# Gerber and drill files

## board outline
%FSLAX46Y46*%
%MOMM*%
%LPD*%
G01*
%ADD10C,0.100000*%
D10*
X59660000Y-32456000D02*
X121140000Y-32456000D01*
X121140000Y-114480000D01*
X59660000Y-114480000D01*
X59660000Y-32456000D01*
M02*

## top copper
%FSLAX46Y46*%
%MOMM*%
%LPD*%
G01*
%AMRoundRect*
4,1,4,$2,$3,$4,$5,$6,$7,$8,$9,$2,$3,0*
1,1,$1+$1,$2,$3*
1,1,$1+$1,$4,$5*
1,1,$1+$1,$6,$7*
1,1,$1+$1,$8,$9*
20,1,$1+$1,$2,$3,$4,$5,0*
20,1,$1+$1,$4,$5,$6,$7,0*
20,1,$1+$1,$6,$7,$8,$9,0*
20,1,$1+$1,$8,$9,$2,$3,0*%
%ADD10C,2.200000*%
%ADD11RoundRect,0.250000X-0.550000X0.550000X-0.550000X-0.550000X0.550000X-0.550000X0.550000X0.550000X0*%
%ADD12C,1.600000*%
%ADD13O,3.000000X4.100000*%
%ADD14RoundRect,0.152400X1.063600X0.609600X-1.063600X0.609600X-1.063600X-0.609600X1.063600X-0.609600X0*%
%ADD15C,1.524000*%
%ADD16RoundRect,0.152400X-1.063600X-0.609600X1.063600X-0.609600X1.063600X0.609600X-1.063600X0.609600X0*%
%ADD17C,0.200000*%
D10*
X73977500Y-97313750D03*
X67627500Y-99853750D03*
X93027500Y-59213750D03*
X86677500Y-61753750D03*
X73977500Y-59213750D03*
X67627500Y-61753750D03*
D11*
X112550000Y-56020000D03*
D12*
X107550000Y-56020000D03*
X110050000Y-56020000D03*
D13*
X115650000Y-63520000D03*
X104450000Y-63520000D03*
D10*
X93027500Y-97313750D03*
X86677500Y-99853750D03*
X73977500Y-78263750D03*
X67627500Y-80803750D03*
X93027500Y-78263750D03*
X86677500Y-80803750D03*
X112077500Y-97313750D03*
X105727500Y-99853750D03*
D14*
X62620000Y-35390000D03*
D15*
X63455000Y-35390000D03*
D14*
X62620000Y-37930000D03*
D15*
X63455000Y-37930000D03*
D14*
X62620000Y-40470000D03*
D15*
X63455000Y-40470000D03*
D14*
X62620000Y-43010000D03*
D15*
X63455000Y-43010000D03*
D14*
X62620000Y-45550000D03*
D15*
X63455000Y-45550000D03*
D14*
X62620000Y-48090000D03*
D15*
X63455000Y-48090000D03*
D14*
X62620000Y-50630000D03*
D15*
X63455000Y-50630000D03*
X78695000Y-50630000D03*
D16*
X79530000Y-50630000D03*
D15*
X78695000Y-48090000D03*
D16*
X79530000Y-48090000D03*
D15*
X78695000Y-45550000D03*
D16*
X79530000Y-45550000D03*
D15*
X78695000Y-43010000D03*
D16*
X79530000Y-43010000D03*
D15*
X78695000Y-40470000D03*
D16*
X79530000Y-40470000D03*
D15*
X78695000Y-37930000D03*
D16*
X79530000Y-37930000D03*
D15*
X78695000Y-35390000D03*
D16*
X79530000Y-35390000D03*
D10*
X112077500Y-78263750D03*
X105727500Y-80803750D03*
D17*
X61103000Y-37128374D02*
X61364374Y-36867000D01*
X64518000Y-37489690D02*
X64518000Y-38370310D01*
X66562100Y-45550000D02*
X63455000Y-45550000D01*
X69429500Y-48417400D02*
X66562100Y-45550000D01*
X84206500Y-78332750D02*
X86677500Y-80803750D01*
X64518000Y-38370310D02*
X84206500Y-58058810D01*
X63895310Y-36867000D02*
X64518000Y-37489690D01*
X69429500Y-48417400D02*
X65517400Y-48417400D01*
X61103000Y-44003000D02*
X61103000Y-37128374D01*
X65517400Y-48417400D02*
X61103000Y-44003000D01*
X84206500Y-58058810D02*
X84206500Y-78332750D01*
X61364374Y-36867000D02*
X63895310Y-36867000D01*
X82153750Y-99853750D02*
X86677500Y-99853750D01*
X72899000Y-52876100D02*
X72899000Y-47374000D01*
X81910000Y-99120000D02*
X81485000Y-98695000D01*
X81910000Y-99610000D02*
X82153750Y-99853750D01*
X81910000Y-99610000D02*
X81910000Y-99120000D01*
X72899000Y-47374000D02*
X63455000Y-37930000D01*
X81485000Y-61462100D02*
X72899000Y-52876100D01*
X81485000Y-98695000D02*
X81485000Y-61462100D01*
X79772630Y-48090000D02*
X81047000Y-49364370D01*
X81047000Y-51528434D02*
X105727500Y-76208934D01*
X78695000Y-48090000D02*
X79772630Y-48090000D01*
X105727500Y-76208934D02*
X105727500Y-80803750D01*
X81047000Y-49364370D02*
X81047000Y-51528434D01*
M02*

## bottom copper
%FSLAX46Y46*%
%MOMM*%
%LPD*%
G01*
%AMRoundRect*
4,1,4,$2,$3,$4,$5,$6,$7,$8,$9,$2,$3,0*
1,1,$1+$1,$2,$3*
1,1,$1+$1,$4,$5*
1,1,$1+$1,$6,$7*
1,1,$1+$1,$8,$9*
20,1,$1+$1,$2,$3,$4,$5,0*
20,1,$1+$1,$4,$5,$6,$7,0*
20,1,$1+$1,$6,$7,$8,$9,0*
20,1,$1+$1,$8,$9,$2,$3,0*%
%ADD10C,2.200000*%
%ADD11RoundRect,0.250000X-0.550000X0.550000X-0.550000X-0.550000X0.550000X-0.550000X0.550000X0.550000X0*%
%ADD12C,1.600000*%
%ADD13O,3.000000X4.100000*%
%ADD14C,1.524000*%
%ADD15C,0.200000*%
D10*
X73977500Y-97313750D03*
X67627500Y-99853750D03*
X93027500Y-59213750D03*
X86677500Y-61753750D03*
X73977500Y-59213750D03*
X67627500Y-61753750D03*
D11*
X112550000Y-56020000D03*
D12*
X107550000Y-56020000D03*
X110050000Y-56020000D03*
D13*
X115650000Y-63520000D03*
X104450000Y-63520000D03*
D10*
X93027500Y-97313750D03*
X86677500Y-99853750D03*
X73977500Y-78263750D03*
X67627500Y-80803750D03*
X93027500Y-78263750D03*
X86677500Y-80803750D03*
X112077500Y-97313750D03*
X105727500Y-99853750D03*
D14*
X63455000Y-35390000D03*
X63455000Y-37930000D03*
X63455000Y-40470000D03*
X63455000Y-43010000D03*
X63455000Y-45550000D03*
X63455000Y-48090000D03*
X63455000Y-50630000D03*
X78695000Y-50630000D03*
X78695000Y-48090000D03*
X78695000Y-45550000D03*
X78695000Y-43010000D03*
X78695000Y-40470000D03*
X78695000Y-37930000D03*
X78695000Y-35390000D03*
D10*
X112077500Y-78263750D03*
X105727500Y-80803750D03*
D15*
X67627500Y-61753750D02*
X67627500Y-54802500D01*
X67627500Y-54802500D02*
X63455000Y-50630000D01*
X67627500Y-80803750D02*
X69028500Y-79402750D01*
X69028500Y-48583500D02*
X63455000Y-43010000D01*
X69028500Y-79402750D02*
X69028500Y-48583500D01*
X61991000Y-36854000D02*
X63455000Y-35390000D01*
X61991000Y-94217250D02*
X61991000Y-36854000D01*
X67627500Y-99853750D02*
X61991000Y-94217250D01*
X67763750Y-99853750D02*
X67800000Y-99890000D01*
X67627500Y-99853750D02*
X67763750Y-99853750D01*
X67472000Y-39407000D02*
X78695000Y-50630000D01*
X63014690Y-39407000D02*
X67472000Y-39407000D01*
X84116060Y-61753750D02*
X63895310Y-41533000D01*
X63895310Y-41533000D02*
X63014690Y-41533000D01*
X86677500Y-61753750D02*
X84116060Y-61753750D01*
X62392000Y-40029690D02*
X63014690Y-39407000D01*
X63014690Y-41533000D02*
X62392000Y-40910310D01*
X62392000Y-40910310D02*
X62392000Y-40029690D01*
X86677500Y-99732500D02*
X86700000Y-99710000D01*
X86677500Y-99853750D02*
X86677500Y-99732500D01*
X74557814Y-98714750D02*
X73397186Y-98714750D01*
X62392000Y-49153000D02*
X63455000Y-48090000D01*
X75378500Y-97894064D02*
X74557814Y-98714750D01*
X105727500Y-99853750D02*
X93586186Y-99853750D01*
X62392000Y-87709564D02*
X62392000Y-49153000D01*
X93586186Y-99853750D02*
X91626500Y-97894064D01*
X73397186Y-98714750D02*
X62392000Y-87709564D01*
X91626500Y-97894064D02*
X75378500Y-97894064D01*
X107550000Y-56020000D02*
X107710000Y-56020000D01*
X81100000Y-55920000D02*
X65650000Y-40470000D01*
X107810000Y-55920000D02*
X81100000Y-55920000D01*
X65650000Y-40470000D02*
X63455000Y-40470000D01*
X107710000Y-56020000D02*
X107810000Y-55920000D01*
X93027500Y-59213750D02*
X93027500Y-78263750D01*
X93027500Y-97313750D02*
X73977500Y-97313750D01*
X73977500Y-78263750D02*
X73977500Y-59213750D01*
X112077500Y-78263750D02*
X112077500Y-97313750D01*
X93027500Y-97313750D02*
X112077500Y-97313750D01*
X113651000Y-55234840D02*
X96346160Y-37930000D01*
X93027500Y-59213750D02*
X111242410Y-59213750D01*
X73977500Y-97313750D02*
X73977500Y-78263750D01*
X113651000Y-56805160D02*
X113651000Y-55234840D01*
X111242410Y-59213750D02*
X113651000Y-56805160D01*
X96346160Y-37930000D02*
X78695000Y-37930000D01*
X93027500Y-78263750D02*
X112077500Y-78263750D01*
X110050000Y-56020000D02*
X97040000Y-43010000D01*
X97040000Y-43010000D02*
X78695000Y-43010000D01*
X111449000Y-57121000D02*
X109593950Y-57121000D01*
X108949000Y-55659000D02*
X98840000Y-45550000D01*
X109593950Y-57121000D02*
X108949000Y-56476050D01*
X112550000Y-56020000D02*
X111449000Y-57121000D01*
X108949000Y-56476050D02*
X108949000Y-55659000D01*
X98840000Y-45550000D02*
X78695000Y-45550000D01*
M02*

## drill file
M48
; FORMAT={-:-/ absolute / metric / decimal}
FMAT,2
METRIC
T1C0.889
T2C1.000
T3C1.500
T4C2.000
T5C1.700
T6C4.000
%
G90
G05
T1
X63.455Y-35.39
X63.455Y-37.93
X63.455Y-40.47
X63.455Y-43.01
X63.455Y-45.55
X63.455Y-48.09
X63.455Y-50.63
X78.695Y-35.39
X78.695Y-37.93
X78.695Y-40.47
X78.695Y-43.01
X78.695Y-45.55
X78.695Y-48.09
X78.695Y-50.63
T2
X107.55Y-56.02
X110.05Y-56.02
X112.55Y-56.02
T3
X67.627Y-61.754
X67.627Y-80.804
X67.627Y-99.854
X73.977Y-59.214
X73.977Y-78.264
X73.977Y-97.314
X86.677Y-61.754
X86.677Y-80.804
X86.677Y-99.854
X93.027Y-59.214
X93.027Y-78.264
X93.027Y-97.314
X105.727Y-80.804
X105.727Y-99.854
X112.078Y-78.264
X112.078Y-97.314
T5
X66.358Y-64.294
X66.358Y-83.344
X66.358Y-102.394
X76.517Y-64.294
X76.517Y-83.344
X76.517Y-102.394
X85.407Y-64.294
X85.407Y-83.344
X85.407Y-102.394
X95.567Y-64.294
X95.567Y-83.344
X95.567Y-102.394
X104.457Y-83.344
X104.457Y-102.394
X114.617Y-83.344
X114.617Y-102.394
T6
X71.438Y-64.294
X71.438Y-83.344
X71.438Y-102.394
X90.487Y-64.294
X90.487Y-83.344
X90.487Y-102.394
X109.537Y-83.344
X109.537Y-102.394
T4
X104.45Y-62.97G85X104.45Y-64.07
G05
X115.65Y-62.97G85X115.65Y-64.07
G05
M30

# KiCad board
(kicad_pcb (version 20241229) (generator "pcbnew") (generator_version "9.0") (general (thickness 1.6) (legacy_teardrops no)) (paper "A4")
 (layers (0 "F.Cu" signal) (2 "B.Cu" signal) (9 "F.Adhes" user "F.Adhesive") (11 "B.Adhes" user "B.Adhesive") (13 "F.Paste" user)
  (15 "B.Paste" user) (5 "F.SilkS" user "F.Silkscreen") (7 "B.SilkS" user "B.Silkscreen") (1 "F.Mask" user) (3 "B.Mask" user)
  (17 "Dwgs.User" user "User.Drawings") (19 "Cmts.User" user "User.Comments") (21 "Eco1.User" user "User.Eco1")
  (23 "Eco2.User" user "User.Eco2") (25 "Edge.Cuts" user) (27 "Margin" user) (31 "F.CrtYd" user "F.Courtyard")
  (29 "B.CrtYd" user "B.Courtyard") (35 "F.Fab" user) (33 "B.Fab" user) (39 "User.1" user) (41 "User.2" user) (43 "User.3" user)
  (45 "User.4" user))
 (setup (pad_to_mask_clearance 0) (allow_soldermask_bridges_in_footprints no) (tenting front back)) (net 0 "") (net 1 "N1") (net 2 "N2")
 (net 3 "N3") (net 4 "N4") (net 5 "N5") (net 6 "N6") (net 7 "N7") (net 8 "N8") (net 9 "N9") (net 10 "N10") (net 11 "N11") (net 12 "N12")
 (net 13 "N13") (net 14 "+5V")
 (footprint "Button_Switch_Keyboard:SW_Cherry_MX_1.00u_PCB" (layer "F.Cu") (at 73.9775 97.31375)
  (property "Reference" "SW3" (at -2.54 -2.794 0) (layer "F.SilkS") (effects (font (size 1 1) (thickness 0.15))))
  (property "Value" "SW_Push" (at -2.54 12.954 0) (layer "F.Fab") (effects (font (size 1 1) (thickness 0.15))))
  (pad "" np_thru_hole circle (at -7.62 5.08) (size 1.7 1.7) (drill 1.7) (layers "*.Cu" "*.Mask"))
  (pad "" np_thru_hole circle (at -2.54 5.08) (size 4 4) (drill 4) (layers "*.Cu" "*.Mask"))
  (pad "" np_thru_hole circle (at 2.54 5.08) (size 1.7 1.7) (drill 1.7) (layers "*.Cu" "*.Mask"))
  (pad "1" thru_hole circle (at 0 0) (size 2.2 2.2) (drill 1.5) (layers "*.Cu" "*.Mask") (remove_unused_layers no) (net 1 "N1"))
  (pad "2" thru_hole circle (at -6.35 2.54) (size 2.2 2.2) (drill 1.5) (layers "*.Cu" "*.Mask") (remove_unused_layers no) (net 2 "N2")))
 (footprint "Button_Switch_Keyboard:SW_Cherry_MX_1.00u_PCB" (layer "F.Cu") (at 93.0275 59.21375)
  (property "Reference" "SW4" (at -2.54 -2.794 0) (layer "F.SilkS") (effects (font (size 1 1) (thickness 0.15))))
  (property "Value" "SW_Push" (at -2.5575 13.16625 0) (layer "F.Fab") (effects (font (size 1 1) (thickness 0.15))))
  (pad "" np_thru_hole circle (at -7.62 5.08) (size 1.7 1.7) (drill 1.7) (layers "*.Cu" "*.Mask"))
  (pad "" np_thru_hole circle (at -2.54 5.08) (size 4 4) (drill 4) (layers "*.Cu" "*.Mask"))
  (pad "" np_thru_hole circle (at 2.54 5.08) (size 1.7 1.7) (drill 1.7) (layers "*.Cu" "*.Mask"))
  (pad "1" thru_hole circle (at 0 0) (size 2.2 2.2) (drill 1.5) (layers "*.Cu" "*.Mask") (remove_unused_layers no) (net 1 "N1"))
  (pad "2" thru_hole circle (at -6.35 2.54) (size 2.2 2.2) (drill 1.5) (layers "*.Cu" "*.Mask") (remove_unused_layers no) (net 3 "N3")))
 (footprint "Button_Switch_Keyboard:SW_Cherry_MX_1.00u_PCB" (layer "F.Cu") (at 73.9775 59.21375)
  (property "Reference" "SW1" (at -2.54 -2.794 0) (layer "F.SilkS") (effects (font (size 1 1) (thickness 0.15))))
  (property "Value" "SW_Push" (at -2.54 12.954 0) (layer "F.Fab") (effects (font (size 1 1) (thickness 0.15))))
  (pad "" np_thru_hole circle (at -7.62 5.08) (size 1.7 1.7) (drill 1.7) (layers "*.Cu" "*.Mask"))
  (pad "" np_thru_hole circle (at -2.54 5.08) (size 4 4) (drill 4) (layers "*.Cu" "*.Mask"))
  (pad "" np_thru_hole circle (at 2.54 5.08) (size 1.7 1.7) (drill 1.7) (layers "*.Cu" "*.Mask"))
  (pad "1" thru_hole circle (at 0 0) (size 2.2 2.2) (drill 1.5) (layers "*.Cu" "*.Mask") (remove_unused_layers no) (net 1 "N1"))
  (pad "2" thru_hole circle (at -6.35 2.54) (size 2.2 2.2) (drill 1.5) (layers "*.Cu" "*.Mask") (remove_unused_layers no) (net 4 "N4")))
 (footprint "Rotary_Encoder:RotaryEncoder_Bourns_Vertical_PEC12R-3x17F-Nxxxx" (layer "F.Cu") (at 112.55 56.02 -90)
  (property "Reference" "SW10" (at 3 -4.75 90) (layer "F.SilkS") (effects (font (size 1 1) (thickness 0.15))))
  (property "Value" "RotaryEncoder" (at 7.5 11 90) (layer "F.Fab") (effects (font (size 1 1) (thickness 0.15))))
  (pad "A" thru_hole roundrect (at 0 0 270) (size 1.6 1.6) (drill 1) (layers "*.Cu" "*.Mask") (remove_unused_layers no)
   (roundrect_rratio 0.15625) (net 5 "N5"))
  (pad "B" thru_hole circle (at 0 5 270) (size 1.6 1.6) (drill 1) (layers "*.Cu" "*.Mask") (remove_unused_layers no) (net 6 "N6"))
  (pad "C" thru_hole circle (at 0 2.5 270) (size 1.6 1.6) (drill 1) (layers "*.Cu" "*.Mask") (remove_unused_layers no) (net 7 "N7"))
  (pad "SH" thru_hole oval (at 7.5 -3.1 270) (size 4.1 3) (drill oval 3.1 2) (layers "*.Cu" "*.Mask") (remove_unused_layers no))
  (pad "SH" thru_hole oval (at 7.5 8.1 270) (size 4.1 3) (drill oval 3.1 2) (layers "*.Cu" "*.Mask") (remove_unused_layers no)))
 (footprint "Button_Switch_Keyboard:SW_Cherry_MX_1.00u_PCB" (layer "F.Cu") (at 93.0275 97.31375)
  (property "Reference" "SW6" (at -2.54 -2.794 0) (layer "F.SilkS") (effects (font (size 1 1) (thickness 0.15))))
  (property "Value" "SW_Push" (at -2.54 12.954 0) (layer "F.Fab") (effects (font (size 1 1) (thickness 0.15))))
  (pad "" np_thru_hole circle (at -7.62 5.08) (size 1.7 1.7) (drill 1.7) (layers "*.Cu" "*.Mask"))
  (pad "" np_thru_hole circle (at -2.54 5.08) (size 4 4) (drill 4) (layers "*.Cu" "*.Mask"))
  (pad "" np_thru_hole circle (at 2.54 5.08) (size 1.7 1.7) (drill 1.7) (layers "*.Cu" "*.Mask"))
  (pad "1" thru_hole circle (at 0 0) (size 2.2 2.2) (drill 1.5) (layers "*.Cu" "*.Mask") (remove_unused_layers no) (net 1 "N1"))
  (pad "2" thru_hole circle (at -6.35 2.54) (size 2.2 2.2) (drill 1.5) (layers "*.Cu" "*.Mask") (remove_unused_layers no) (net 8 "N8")))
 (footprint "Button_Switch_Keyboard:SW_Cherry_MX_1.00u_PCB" (layer "F.Cu") (at 73.9775 78.26375)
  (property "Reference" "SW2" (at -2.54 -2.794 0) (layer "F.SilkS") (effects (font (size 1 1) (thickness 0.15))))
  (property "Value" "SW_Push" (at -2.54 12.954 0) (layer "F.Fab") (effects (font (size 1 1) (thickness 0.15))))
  (pad "" np_thru_hole circle (at -7.62 5.08) (size 1.7 1.7) (drill 1.7) (layers "*.Cu" "*.Mask"))
  (pad "" np_thru_hole circle (at -2.54 5.08) (size 4 4) (drill 4) (layers "*.Cu" "*.Mask"))
  (pad "" np_thru_hole circle (at 2.54 5.08) (size 1.7 1.7) (drill 1.7) (layers "*.Cu" "*.Mask"))
  (pad "1" thru_hole circle (at 0 0) (size 2.2 2.2) (drill 1.5) (layers "*.Cu" "*.Mask") (remove_unused_layers no) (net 1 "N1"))
  (pad "2" thru_hole circle (at -6.35 2.54) (size 2.2 2.2) (drill 1.5) (layers "*.Cu" "*.Mask") (remove_unused_layers no) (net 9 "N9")))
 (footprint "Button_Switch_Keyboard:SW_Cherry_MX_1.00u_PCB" (layer "F.Cu") (at 93.0275 78.26375)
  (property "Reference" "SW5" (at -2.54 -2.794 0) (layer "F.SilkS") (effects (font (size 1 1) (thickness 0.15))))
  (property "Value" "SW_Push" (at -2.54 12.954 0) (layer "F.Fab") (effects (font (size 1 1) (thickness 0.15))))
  (pad "" np_thru_hole circle (at -7.62 5.08) (size 1.7 1.7) (drill 1.7) (layers "*.Cu" "*.Mask"))
  (pad "" np_thru_hole circle (at -2.54 5.08) (size 4 4) (drill 4) (layers "*.Cu" "*.Mask"))
  (pad "" np_thru_hole circle (at 2.54 5.08) (size 1.7 1.7) (drill 1.7) (layers "*.Cu" "*.Mask"))
  (pad "1" thru_hole circle (at 0 0) (size 2.2 2.2) (drill 1.5) (layers "*.Cu" "*.Mask") (remove_unused_layers no) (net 1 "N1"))
  (pad "2" thru_hole circle (at -6.35 2.54) (size 2.2 2.2) (drill 1.5) (layers "*.Cu" "*.Mask") (remove_unused_layers no) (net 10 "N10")))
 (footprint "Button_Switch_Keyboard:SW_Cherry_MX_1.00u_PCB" (layer "F.Cu") (at 112.0775 97.31375)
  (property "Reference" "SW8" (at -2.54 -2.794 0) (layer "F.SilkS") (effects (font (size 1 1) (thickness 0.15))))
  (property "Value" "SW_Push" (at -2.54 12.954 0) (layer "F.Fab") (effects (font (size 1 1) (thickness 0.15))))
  (pad "" np_thru_hole circle (at -7.62 5.08) (size 1.7 1.7) (drill 1.7) (layers "*.Cu" "*.Mask"))
  (pad "" np_thru_hole circle (at -2.54 5.08) (size 4 4) (drill 4) (layers "*.Cu" "*.Mask"))
  (pad "" np_thru_hole circle (at 2.54 5.08) (size 1.7 1.7) (drill 1.7) (layers "*.Cu" "*.Mask"))
  (pad "1" thru_hole circle (at 0 0) (size 2.2 2.2) (drill 1.5) (layers "*.Cu" "*.Mask") (remove_unused_layers no) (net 1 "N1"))
  (pad "2" thru_hole circle (at -6.35 2.54) (size 2.2 2.2) (drill 1.5) (layers "*.Cu" "*.Mask") (remove_unused_layers no) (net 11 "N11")))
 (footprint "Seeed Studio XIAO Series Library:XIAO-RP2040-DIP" (layer "F.Cu") (at 71.075 43.01)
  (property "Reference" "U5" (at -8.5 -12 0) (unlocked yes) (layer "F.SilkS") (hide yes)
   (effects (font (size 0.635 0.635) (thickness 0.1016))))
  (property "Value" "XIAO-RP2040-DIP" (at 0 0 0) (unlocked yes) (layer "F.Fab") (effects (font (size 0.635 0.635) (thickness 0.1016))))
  (pad "1" smd roundrect (at -8.455 -7.62 180) (size 2.432 1.524) (layers "F.Cu" "F.Mask") (roundrect_rratio 0.1) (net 2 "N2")
   (thermal_bridge_angle 45))
  (pad "1" thru_hole circle (at -7.62 -7.62 180) (size 1.524 1.524) (drill 0.889) (layers "*.Cu" "*.Mask") (remove_unused_layers no)
   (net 2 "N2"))
  (pad "2" smd roundrect (at -8.455 -5.08 180) (size 2.432 1.524) (layers "F.Cu" "F.Mask") (roundrect_rratio 0.1) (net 8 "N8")
   (thermal_bridge_angle 45))
  (pad "2" thru_hole circle (at -7.62 -5.08 180) (size 1.524 1.524) (drill 0.889) (layers "*.Cu" "*.Mask") (remove_unused_layers no)
   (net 8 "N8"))
  (pad "3" smd roundrect (at -8.455 -2.54 180) (size 2.432 1.524) (layers "F.Cu" "F.Mask") (roundrect_rratio 0.1) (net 6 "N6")
   (thermal_bridge_angle 45))
  (pad "3" thru_hole circle (at -7.62 -2.54 180) (size 1.524 1.524) (drill 0.889) (layers "*.Cu" "*.Mask") (remove_unused_layers no)
   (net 6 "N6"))
  (pad "4" smd roundrect (at -8.455 0 180) (size 2.432 1.524) (layers "F.Cu" "F.Mask") (roundrect_rratio 0.1) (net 9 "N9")
   (thermal_bridge_angle 45))
  (pad "4" thru_hole circle (at -7.62 0 180) (size 1.524 1.524) (drill 0.889) (layers "*.Cu" "*.Mask") (remove_unused_layers no)
   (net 9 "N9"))
  (pad "5" smd roundrect (at -8.455 2.54 180) (size 2.432 1.524) (layers "F.Cu" "F.Mask") (roundrect_rratio 0.1) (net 10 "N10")
   (thermal_bridge_angle 45))
  (pad "5" thru_hole circle (at -7.62 2.54 180) (size 1.524 1.524) (drill 0.889) (layers "*.Cu" "*.Mask") (remove_unused_layers no)
   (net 10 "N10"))
  (pad "6" smd roundrect (at -8.455 5.08 180) (size 2.432 1.524) (layers "F.Cu" "F.Mask") (roundrect_rratio 0.1) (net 11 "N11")
   (thermal_bridge_angle 45))
  (pad "6" thru_hole circle (at -7.62 5.08 180) (size 1.524 1.524) (drill 0.889) (layers "*.Cu" "*.Mask") (remove_unused_layers no)
   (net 11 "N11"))
  (pad "7" smd roundrect (at -8.455 7.62 180) (size 2.432 1.524) (layers "F.Cu" "F.Mask") (roundrect_rratio 0.1) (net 4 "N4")
   (thermal_bridge_angle 45))
  (pad "7" thru_hole circle (at -7.62 7.62 180) (size 1.524 1.524) (drill 0.889) (layers "*.Cu" "*.Mask") (remove_unused_layers no)
   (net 4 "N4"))
  (pad "8" thru_hole circle (at 7.62 7.62) (size 1.524 1.524) (drill 0.889) (layers "*.Cu" "*.Mask") (remove_unused_layers no) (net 3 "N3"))
  (pad "8" smd roundrect (at 8.455 7.62) (size 2.432 1.524) (layers "F.Cu" "F.Mask") (roundrect_rratio 0.1) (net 3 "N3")
   (thermal_bridge_angle 45))
  (pad "9" thru_hole circle (at 7.62 5.08) (size 1.524 1.524) (drill 0.889) (layers "*.Cu" "*.Mask") (remove_unused_layers no)
   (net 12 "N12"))
  (pad "9" smd roundrect (at 8.455 5.08) (size 2.432 1.524) (layers "F.Cu" "F.Mask") (roundrect_rratio 0.1) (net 12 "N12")
   (thermal_bridge_angle 45))
  (pad "10" thru_hole circle (at 7.62 2.54) (size 1.524 1.524) (drill 0.889) (layers "*.Cu" "*.Mask") (remove_unused_layers no) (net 5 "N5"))
  (pad "10" smd roundrect (at 8.455 2.54) (size 2.432 1.524) (layers "F.Cu" "F.Mask") (roundrect_rratio 0.1) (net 5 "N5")
   (thermal_bridge_angle 45))
  (pad "11" thru_hole circle (at 7.62 0) (size 1.524 1.524) (drill 0.889) (layers "*.Cu" "*.Mask") (remove_unused_layers no) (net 7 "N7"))
  (pad "11" smd roundrect (at 8.455 0) (size 2.432 1.524) (layers "F.Cu" "F.Mask") (roundrect_rratio 0.1) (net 7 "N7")
   (thermal_bridge_angle 45))
  (pad "12" thru_hole circle (at 7.62 -2.54) (size 1.524 1.524) (drill 0.889) (layers "*.Cu" "*.Mask") (remove_unused_layers no)
   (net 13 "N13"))
  (pad "12" smd roundrect (at 8.455 -2.54) (size 2.432 1.524) (layers "F.Cu" "F.Mask") (roundrect_rratio 0.1) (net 13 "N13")
   (thermal_bridge_angle 45))
  (pad "13" thru_hole circle (at 7.62 -5.08) (size 1.524 1.524) (drill 0.889) (layers "*.Cu" "*.Mask") (remove_unused_layers no)
   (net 1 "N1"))
  (pad "13" smd roundrect (at 8.455 -5.08) (size 2.432 1.524) (layers "F.Cu" "F.Mask") (roundrect_rratio 0.1) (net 1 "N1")
   (thermal_bridge_angle 45))
  (pad "14" thru_hole circle (at 7.62 -7.62) (size 1.524 1.524) (drill 0.889) (layers "*.Cu" "*.Mask") (remove_unused_layers no)
   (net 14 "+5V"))
  (pad "14" smd roundrect (at 8.455 -7.62) (size 2.432 1.524) (layers "F.Cu" "F.Mask") (roundrect_rratio 0.1) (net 14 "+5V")
   (thermal_bridge_angle 45)))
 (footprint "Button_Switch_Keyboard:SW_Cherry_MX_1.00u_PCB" (layer "F.Cu") (at 112.0775 78.26375)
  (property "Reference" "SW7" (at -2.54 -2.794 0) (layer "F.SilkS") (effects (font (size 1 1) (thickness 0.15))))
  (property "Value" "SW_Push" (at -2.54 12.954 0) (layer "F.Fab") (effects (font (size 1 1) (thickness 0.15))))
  (pad "" np_thru_hole circle (at -7.62 5.08) (size 1.7 1.7) (drill 1.7) (layers "*.Cu" "*.Mask"))
  (pad "" np_thru_hole circle (at -2.54 5.08) (size 4 4) (drill 4) (layers "*.Cu" "*.Mask"))
  (pad "" np_thru_hole circle (at 2.54 5.08) (size 1.7 1.7) (drill 1.7) (layers "*.Cu" "*.Mask"))
  (pad "1" thru_hole circle (at 0 0) (size 2.2 2.2) (drill 1.5) (layers "*.Cu" "*.Mask") (remove_unused_layers no) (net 1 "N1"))
  (pad "2" thru_hole circle (at -6.35 2.54) (size 2.2 2.2) (drill 1.5) (layers "*.Cu" "*.Mask") (remove_unused_layers no) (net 12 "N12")))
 (gr_rect (start 59.66 32.456) (end 121.14 114.48) (stroke (width 0.1) (type solid)) (fill no) (layer "Edge.Cuts"))
 (segment (start 67.6275 61.75375) (end 67.6275 54.8025) (width 0.2) (layer "B.Cu") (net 4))
 (segment (start 67.6275 54.8025) (end 63.455 50.63) (width 0.2) (layer "B.Cu") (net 4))
 (segment (start 67.6275 80.80375) (end 69.0285 79.40275) (width 0.2) (layer "B.Cu") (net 9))
 (segment (start 69.0285 48.5835) (end 63.455 43.01) (width 0.2) (layer "B.Cu") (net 9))
 (segment (start 69.0285 79.40275) (end 69.0285 48.5835) (width 0.2) (layer "B.Cu") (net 9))
 (segment (start 61.991 36.854) (end 63.455 35.39) (width 0.2) (layer "B.Cu") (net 2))
 (segment (start 61.991 94.21725) (end 61.991 36.854) (width 0.2) (layer "B.Cu") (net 2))
 (segment (start 67.6275 99.85375) (end 61.991 94.21725) (width 0.2) (layer "B.Cu") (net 2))
 (segment (start 67.76375 99.85375) (end 67.8 99.89) (width 0.2) (layer "B.Cu") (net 2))
 (segment (start 67.6275 99.85375) (end 67.76375 99.85375) (width 0.2) (layer "B.Cu") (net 2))
 (segment (start 67.472 39.407) (end 78.695 50.63) (width 0.2) (layer "B.Cu") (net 3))
 (segment (start 63.01469 39.407) (end 67.472 39.407) (width 0.2) (layer "B.Cu") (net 3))
 (segment (start 84.11606 61.75375) (end 63.89531 41.533) (width 0.2) (layer "B.Cu") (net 3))
 (segment (start 63.89531 41.533) (end 63.01469 41.533) (width 0.2) (layer "B.Cu") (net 3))
 (segment (start 86.6775 61.75375) (end 84.11606 61.75375) (width 0.2) (layer "B.Cu") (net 3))
 (segment (start 62.392 40.02969) (end 63.01469 39.407) (width 0.2) (layer "B.Cu") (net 3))
 (segment (start 63.01469 41.533) (end 62.392 40.91031) (width 0.2) (layer "B.Cu") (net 3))
 (segment (start 62.392 40.91031) (end 62.392 40.02969) (width 0.2) (layer "B.Cu") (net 3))
 (segment (start 61.103 37.128374) (end 61.364374 36.867) (width 0.2) (layer "F.Cu") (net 10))
 (segment (start 64.518 37.48969) (end 64.518 38.37031) (width 0.2) (layer "F.Cu") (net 10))
 (segment (start 66.5621 45.55) (end 63.455 45.55) (width 0.2) (layer "F.Cu") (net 10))
 (segment (start 69.4295 48.4174) (end 66.5621 45.55) (width 0.2) (layer "F.Cu") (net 10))
 (segment (start 84.2065 78.33275) (end 86.6775 80.80375) (width 0.2) (layer "F.Cu") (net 10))
 (segment (start 64.518 38.37031) (end 84.2065 58.05881) (width 0.2) (layer "F.Cu") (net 10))
 (segment (start 63.89531 36.867) (end 64.518 37.48969) (width 0.2) (layer "F.Cu") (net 10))
 (segment (start 69.4295 48.4174) (end 65.5174 48.4174) (width 0.2) (layer "F.Cu") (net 10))
 (segment (start 61.103 44.003) (end 61.103 37.128374) (width 0.2) (layer "F.Cu") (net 10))
 (segment (start 65.5174 48.4174) (end 61.103 44.003) (width 0.2) (layer "F.Cu") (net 10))
 (segment (start 84.2065 58.05881) (end 84.2065 78.33275) (width 0.2) (layer "F.Cu") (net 10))
 (segment (start 61.364374 36.867) (end 63.89531 36.867) (width 0.2) (layer "F.Cu") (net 10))
 (segment (start 82.15375 99.85375) (end 86.6775 99.85375) (width 0.2) (layer "F.Cu") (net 8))
 (segment (start 72.899 52.8761) (end 72.899 47.374) (width 0.2) (layer "F.Cu") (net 8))
 (segment (start 81.91 99.12) (end 81.485 98.695) (width 0.2) (layer "F.Cu") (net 8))
 (segment (start 81.91 99.61) (end 82.15375 99.85375) (width 0.2) (layer "F.Cu") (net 8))
 (segment (start 81.91 99.61) (end 81.91 99.12) (width 0.2) (layer "F.Cu") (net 8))
 (segment (start 72.899 47.374) (end 63.455 37.93) (width 0.2) (layer "F.Cu") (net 8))
 (segment (start 81.485 61.4621) (end 72.899 52.8761) (width 0.2) (layer "F.Cu") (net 8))
 (segment (start 81.485 98.695) (end 81.485 61.4621) (width 0.2) (layer "F.Cu") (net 8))
 (segment (start 86.6775 99.7325) (end 86.7 99.71) (width 0.2) (layer "B.Cu") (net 8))
 (segment (start 86.6775 99.85375) (end 86.6775 99.7325) (width 0.2) (layer "B.Cu") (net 8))
 (segment (start 79.77263 48.09) (end 81.047 49.36437) (width 0.2) (layer "F.Cu") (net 12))
 (segment (start 81.047 51.528434) (end 105.7275 76.208934) (width 0.2) (layer "F.Cu") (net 12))
 (segment (start 78.695 48.09) (end 79.77263 48.09) (width 0.2) (layer "F.Cu") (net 12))
 (segment (start 105.7275 76.208934) (end 105.7275 80.80375) (width 0.2) (layer "F.Cu") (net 12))
 (segment (start 81.047 49.36437) (end 81.047 51.528434) (width 0.2) (layer "F.Cu") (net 12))
 (segment (start 74.557814 98.71475) (end 73.397186 98.71475) (width 0.2) (layer "B.Cu") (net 11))
 (segment (start 62.392 49.153) (end 63.455 48.09) (width 0.2) (layer "B.Cu") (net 11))
 (segment (start 75.3785 97.894064) (end 74.557814 98.71475) (width 0.2) (layer "B.Cu") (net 11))
 (segment (start 105.7275 99.85375) (end 93.586186 99.85375) (width 0.2) (layer "B.Cu") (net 11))
 (segment (start 62.392 87.709564) (end 62.392 49.153) (width 0.2) (layer "B.Cu") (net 11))
 (segment (start 93.586186 99.85375) (end 91.6265 97.894064) (width 0.2) (layer "B.Cu") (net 11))
 (segment (start 73.397186 98.71475) (end 62.392 87.709564) (width 0.2) (layer "B.Cu") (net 11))
 (segment (start 91.6265 97.894064) (end 75.3785 97.894064) (width 0.2) (layer "B.Cu") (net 11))
 (segment (start 107.55 56.02) (end 107.71 56.02) (width 0.2) (layer "B.Cu") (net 6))
 (segment (start 81.1 55.92) (end 65.65 40.47) (width 0.2) (layer "B.Cu") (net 6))
 (segment (start 107.81 55.92) (end 81.1 55.92) (width 0.2) (layer "B.Cu") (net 6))
 (segment (start 65.65 40.47) (end 63.455 40.47) (width 0.2) (layer "B.Cu") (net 6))
 (segment (start 107.71 56.02) (end 107.81 55.92) (width 0.2) (layer "B.Cu") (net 6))
 (segment (start 93.0275 59.21375) (end 93.0275 78.26375) (width 0.2) (layer "B.Cu") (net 1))
 (segment (start 93.0275 97.31375) (end 73.9775 97.31375) (width 0.2) (layer "B.Cu") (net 1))
 (segment (start 73.9775 78.26375) (end 73.9775 59.21375) (width 0.2) (layer "B.Cu") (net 1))
 (segment (start 112.0775 78.26375) (end 112.0775 97.31375) (width 0.2) (layer "B.Cu") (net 1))
 (segment (start 93.0275 97.31375) (end 112.0775 97.31375) (width 0.2) (layer "B.Cu") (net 1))
 (segment (start 113.651 55.23484) (end 96.34616 37.93) (width 0.2) (layer "B.Cu") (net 1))
 (segment (start 93.0275 59.21375) (end 111.24241 59.21375) (width 0.2) (layer "B.Cu") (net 1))
 (segment (start 73.9775 97.31375) (end 73.9775 78.26375) (width 0.2) (layer "B.Cu") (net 1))
 (segment (start 113.651 56.80516) (end 113.651 55.23484) (width 0.2) (layer "B.Cu") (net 1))
 (segment (start 111.24241 59.21375) (end 113.651 56.80516) (width 0.2) (layer "B.Cu") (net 1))
 (segment (start 96.34616 37.93) (end 78.695 37.93) (width 0.2) (layer "B.Cu") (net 1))
 (segment (start 93.0275 78.26375) (end 112.0775 78.26375) (width 0.2) (layer "B.Cu") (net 1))
 (segment (start 110.05 56.02) (end 97.04 43.01) (width 0.2) (layer "B.Cu") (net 7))
 (segment (start 97.04 43.01) (end 78.695 43.01) (width 0.2) (layer "B.Cu") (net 7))
 (segment (start 111.449 57.121) (end 109.59395 57.121) (width 0.2) (layer "B.Cu") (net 5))
 (segment (start 108.949 55.659) (end 98.84 45.55) (width 0.2) (layer "B.Cu") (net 5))
 (segment (start 109.59395 57.121) (end 108.949 56.47605) (width 0.2) (layer "B.Cu") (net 5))
 (segment (start 112.55 56.02) (end 111.449 57.121) (width 0.2) (layer "B.Cu") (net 5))
 (segment (start 108.949 56.47605) (end 108.949 55.659) (width 0.2) (layer "B.Cu") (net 5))
 (segment (start 98.84 45.55) (end 78.695 45.55) (width 0.2) (layer "B.Cu") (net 5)))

